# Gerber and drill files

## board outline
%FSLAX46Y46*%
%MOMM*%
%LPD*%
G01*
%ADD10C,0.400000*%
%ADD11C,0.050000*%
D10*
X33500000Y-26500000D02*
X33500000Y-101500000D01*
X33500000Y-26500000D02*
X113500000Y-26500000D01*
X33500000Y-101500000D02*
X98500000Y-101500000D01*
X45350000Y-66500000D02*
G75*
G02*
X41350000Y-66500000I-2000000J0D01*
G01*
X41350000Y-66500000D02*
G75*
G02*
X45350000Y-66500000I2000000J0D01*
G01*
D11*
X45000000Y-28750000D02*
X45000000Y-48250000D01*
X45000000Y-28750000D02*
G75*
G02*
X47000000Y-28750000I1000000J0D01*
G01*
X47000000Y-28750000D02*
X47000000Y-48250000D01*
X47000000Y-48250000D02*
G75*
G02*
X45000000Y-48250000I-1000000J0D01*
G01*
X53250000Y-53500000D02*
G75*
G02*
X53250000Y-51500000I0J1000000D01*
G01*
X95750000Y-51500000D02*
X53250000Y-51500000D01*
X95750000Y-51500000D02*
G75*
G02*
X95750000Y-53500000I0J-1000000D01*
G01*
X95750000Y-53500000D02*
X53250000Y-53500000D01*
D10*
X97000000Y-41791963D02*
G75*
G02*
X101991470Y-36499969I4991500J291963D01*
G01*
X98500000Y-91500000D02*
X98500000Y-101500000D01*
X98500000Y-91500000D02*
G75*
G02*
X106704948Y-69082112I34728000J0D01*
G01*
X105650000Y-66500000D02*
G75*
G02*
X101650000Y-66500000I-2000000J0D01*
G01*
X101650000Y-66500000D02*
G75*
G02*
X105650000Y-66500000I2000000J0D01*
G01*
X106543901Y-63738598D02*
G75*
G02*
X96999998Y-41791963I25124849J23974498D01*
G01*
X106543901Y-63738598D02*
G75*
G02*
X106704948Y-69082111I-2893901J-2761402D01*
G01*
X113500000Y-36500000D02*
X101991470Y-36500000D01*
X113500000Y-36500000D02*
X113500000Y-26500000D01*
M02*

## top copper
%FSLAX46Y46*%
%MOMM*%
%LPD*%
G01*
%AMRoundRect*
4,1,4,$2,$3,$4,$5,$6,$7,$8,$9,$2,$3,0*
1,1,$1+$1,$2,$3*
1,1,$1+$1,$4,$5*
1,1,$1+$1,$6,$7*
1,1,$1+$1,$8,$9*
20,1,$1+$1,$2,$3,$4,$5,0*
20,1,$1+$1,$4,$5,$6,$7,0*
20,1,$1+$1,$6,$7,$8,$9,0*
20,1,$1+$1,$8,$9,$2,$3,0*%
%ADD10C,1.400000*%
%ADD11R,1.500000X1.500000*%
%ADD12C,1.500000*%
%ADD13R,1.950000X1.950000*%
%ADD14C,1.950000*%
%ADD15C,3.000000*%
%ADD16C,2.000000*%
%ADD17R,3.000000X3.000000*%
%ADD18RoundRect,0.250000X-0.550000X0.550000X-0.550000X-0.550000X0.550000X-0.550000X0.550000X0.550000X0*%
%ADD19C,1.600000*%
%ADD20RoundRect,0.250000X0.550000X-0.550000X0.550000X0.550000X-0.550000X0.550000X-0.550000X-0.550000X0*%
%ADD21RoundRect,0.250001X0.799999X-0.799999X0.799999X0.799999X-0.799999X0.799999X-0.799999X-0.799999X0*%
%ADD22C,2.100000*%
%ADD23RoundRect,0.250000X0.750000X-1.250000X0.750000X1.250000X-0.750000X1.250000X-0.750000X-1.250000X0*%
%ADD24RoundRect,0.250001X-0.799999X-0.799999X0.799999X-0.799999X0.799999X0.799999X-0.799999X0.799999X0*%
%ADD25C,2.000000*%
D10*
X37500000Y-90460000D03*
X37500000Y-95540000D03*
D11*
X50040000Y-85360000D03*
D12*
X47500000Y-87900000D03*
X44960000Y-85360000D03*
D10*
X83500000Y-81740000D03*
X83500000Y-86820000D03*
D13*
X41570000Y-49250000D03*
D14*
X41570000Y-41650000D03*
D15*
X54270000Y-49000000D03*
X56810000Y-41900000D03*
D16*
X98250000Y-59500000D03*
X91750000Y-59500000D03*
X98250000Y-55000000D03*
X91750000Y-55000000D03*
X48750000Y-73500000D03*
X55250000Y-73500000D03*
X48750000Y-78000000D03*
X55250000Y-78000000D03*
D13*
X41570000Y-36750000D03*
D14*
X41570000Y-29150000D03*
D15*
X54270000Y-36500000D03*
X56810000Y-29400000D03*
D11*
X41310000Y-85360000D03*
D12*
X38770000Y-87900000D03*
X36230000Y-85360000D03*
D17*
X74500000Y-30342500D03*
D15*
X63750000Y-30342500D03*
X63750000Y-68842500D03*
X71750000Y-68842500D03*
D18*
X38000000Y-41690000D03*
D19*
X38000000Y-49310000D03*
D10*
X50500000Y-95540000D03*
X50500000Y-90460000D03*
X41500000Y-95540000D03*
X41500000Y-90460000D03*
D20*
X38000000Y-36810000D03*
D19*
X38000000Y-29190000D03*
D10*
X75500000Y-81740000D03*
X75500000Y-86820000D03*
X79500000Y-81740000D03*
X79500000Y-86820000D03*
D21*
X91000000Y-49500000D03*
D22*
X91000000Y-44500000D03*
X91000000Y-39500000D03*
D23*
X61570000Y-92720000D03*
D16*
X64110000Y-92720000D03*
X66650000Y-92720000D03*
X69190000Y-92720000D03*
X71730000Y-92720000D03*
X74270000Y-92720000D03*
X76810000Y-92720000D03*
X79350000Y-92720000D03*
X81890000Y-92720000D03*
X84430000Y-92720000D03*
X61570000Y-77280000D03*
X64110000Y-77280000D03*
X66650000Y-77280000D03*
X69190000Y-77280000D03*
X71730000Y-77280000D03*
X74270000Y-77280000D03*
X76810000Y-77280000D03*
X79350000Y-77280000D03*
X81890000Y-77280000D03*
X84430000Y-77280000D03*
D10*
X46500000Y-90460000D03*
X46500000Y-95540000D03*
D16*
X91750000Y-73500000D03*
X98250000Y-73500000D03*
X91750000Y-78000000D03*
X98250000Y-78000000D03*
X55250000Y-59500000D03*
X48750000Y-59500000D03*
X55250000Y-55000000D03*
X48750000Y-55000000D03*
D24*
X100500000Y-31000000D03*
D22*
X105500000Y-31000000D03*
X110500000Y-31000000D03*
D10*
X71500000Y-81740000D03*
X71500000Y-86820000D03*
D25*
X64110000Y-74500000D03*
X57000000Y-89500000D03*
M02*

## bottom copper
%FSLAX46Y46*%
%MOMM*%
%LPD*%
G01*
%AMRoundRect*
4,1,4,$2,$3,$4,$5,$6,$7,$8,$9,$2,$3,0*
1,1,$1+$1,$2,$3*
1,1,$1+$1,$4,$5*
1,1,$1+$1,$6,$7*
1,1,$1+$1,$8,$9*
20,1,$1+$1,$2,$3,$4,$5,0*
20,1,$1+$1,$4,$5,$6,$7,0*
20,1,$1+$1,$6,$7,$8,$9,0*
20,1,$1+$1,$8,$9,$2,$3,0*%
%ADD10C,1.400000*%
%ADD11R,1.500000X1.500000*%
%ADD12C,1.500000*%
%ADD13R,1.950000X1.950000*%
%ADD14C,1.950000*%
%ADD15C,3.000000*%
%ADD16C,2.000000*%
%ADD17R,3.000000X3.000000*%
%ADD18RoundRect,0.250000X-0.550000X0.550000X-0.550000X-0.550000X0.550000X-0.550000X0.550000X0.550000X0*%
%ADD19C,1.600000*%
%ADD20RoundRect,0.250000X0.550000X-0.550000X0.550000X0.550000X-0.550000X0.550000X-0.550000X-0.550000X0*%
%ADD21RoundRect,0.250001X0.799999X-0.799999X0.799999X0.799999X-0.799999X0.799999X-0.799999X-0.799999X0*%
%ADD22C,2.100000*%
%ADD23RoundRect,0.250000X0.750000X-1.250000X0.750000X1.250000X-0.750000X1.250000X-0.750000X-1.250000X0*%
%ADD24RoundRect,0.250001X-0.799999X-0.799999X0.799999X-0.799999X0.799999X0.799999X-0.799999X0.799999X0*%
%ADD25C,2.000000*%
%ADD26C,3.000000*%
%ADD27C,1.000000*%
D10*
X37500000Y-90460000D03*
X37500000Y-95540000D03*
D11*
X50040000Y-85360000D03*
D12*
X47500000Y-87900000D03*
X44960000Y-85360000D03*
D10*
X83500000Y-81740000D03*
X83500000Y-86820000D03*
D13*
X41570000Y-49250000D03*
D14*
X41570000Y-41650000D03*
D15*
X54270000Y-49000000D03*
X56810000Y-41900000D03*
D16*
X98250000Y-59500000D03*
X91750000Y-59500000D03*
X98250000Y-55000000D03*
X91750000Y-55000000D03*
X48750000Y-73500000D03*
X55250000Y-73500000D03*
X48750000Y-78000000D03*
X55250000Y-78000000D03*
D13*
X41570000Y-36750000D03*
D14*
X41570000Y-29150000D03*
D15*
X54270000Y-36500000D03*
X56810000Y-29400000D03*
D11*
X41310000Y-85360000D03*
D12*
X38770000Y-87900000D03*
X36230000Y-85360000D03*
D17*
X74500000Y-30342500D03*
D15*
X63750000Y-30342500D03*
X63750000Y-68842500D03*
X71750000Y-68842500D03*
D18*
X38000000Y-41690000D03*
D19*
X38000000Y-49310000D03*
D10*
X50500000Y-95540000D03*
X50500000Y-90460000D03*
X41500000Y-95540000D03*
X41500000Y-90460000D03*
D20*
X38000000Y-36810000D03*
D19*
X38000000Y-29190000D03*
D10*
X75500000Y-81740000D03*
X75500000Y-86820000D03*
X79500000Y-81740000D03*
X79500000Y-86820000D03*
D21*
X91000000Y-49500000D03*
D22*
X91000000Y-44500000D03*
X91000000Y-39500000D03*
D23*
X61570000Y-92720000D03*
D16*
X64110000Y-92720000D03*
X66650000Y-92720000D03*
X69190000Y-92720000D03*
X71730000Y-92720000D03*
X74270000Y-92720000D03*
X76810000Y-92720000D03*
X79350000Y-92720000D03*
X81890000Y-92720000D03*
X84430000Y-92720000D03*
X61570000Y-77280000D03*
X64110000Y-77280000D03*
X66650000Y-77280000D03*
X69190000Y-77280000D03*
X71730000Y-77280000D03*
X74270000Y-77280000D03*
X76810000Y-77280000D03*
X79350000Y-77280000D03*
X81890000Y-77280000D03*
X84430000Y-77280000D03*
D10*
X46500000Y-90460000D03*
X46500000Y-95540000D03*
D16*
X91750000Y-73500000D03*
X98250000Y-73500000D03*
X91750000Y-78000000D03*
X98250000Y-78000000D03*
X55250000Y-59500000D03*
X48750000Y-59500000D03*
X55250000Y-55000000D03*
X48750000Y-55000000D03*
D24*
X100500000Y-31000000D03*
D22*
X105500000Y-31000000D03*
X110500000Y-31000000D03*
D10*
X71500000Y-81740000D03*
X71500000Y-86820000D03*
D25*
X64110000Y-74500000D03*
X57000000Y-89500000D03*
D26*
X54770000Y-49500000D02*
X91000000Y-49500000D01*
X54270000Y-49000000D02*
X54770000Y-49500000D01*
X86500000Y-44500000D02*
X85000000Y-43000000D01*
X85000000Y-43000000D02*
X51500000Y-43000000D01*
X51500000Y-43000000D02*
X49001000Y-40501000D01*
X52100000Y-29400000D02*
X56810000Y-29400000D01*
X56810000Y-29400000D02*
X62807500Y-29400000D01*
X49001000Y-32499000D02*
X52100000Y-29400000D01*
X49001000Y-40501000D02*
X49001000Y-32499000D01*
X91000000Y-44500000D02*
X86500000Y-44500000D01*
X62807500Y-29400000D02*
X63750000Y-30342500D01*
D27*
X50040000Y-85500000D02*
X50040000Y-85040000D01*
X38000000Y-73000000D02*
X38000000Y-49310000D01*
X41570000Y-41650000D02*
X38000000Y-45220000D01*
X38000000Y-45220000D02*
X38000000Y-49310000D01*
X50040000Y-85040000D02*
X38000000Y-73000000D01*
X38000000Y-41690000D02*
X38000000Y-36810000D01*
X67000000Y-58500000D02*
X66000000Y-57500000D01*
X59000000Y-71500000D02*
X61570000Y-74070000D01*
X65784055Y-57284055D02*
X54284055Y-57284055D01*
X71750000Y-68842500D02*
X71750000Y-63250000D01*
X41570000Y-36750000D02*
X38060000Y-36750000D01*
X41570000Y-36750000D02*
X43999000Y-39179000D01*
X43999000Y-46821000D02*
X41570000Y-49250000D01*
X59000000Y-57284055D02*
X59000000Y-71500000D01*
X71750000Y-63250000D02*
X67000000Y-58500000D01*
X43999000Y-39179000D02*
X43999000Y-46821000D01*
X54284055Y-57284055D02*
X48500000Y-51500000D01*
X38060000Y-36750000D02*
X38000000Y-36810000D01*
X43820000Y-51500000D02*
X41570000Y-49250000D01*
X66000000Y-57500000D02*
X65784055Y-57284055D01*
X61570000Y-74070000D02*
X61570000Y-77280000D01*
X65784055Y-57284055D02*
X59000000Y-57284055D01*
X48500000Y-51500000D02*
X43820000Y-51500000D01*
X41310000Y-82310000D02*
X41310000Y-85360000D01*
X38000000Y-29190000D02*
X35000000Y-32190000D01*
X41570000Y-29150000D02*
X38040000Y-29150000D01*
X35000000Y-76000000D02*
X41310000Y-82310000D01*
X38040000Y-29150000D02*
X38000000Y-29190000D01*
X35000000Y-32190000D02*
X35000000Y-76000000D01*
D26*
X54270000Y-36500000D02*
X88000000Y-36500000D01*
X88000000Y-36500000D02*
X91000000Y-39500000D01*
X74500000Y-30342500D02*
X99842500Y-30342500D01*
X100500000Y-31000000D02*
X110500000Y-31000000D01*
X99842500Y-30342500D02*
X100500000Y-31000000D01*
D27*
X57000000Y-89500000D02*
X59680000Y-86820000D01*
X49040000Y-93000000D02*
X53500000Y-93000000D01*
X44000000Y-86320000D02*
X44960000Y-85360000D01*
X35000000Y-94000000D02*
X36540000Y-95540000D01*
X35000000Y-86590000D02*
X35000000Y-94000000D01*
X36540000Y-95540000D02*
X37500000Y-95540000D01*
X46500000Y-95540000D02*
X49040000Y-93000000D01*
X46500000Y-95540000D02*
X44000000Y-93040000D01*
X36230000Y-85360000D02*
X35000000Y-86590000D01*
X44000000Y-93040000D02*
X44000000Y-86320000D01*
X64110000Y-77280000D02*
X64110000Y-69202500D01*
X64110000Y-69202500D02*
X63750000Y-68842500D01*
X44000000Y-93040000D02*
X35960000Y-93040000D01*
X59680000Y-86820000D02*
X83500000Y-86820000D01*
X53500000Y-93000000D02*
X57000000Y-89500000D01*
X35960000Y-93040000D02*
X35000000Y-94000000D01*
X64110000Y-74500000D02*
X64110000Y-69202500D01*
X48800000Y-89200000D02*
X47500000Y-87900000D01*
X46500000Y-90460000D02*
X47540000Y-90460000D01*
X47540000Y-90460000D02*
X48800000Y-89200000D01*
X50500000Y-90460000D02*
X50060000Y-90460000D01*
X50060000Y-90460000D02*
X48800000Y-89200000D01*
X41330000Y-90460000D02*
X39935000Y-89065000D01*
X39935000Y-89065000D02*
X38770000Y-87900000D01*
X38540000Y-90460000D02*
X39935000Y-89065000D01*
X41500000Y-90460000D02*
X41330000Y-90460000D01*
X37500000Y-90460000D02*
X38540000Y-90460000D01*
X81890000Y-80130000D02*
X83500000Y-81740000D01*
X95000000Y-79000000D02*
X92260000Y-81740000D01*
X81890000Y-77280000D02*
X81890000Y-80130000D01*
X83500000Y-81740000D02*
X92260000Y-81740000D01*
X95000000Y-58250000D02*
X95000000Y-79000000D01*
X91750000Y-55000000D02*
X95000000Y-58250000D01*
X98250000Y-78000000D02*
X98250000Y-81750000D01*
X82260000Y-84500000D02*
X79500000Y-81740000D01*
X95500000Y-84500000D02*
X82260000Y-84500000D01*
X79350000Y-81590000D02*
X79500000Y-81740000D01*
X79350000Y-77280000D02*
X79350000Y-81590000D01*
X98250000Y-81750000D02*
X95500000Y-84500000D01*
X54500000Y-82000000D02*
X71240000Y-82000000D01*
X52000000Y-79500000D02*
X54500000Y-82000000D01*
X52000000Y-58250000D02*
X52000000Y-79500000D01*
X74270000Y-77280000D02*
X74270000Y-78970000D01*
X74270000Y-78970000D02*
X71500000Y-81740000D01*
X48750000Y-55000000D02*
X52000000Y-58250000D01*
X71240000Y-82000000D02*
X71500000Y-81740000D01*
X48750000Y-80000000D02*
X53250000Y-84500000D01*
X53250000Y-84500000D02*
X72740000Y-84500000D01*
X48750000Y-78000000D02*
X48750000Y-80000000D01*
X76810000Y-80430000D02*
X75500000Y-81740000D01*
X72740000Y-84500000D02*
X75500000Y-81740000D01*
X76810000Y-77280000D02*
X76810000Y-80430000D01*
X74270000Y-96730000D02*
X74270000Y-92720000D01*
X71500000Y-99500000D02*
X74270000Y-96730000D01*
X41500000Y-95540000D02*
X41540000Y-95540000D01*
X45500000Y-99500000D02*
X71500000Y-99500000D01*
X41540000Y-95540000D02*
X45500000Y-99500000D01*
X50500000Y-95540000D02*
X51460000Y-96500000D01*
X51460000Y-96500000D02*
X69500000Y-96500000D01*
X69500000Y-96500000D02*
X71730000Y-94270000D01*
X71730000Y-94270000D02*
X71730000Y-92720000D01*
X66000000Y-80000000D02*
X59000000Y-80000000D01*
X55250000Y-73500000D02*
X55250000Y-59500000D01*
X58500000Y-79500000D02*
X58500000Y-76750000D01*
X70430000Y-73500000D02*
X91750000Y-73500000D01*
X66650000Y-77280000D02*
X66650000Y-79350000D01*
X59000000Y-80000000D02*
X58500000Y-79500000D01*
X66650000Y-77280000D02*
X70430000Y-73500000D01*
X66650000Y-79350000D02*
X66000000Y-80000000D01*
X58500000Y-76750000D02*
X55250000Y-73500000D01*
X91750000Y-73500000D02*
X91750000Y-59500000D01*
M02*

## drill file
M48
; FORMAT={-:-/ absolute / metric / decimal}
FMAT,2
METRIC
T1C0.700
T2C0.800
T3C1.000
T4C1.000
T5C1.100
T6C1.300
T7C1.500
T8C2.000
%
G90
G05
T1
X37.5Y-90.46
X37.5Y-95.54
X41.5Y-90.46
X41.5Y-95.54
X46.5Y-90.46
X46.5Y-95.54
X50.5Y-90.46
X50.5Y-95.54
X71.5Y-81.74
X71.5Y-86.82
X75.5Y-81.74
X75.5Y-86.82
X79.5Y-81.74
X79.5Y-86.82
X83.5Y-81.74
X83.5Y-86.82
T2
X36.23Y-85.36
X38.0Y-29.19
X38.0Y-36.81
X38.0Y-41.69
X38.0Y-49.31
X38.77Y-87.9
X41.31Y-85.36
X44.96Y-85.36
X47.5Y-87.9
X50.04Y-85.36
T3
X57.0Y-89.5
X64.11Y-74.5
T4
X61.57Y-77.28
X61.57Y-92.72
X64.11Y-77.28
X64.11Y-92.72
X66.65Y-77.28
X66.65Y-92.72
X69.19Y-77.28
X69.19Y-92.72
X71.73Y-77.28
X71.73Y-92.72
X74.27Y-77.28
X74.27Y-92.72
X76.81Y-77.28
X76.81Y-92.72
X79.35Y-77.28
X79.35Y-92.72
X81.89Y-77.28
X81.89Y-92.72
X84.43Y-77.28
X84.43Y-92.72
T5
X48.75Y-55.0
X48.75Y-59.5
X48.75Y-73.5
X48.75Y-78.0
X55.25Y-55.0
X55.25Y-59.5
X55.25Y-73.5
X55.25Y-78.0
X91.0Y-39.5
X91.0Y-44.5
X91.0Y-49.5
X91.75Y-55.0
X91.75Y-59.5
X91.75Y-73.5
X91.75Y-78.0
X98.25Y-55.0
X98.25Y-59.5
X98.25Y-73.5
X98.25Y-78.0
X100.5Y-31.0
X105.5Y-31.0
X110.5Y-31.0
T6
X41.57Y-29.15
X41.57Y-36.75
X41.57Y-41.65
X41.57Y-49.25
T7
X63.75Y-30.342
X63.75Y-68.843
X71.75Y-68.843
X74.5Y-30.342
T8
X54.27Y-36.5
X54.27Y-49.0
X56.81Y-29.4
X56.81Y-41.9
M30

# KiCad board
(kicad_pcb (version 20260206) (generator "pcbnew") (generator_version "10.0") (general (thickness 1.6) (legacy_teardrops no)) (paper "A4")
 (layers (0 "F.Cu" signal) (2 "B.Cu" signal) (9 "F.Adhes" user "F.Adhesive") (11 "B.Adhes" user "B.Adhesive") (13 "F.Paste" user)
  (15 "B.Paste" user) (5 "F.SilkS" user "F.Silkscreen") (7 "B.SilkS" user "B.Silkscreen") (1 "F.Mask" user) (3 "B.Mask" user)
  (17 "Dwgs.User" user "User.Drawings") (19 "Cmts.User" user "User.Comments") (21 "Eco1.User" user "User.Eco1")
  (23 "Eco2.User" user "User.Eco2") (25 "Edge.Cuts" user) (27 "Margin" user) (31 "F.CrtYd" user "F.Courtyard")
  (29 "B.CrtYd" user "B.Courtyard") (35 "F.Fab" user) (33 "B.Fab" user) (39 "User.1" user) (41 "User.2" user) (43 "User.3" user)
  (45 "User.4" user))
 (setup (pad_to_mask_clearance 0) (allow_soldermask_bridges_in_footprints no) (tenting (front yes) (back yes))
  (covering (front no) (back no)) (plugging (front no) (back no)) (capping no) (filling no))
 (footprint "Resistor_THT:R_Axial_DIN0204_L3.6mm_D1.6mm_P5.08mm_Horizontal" (layer "F.Cu") (at 37.5 90.46 -90)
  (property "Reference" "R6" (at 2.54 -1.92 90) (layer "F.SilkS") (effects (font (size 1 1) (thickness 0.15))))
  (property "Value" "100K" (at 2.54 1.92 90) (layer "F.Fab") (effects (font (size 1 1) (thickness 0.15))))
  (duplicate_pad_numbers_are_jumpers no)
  (pad "1" thru_hole circle (at 0 0 270) (size 1.4 1.4) (drill 0.7) (layers "*.Cu" "*.Mask") (remove_unused_layers no) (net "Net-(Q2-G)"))
  (pad "2" thru_hole circle (at 5.08 0 270) (size 1.4 1.4) (drill 0.7) (layers "*.Cu" "*.Mask") (remove_unused_layers no) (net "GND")))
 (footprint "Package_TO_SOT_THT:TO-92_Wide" (layer "F.Cu") (at 50.04 85.36 180)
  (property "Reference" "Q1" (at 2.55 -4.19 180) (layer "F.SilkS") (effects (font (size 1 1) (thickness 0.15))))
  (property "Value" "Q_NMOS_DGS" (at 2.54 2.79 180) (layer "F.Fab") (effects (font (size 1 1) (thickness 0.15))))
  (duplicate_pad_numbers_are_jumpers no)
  (pad "1" thru_hole rect (at 0 0 180) (size 1.5 1.5) (drill 0.8) (layers "*.Cu" "*.Mask") (remove_unused_layers no) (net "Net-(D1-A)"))
  (pad "2" thru_hole circle (at 2.54 -2.54 180) (size 1.5 1.5) (drill 0.8) (layers "*.Cu" "*.Mask") (remove_unused_layers no)
   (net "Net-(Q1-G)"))
  (pad "3" thru_hole circle (at 5.08 0 180) (size 1.5 1.5) (drill 0.8) (layers "*.Cu" "*.Mask") (remove_unused_layers no) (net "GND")))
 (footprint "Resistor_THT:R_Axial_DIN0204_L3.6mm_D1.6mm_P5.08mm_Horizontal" (layer "F.Cu") (at 83.5 81.74 -90)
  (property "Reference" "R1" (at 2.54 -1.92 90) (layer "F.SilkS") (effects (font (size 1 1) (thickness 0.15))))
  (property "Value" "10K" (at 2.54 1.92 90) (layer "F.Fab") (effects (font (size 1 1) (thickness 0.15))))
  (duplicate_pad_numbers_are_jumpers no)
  (pad "1" thru_hole circle (at 0 0 270) (size 1.4 1.4) (drill 0.7) (layers "*.Cu" "*.Mask") (remove_unused_layers no) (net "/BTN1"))
  (pad "2" thru_hole circle (at 5.08 0 270) (size 1.4 1.4) (drill 0.7) (layers "*.Cu" "*.Mask") (remove_unused_layers no) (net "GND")))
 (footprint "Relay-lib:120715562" (layer "F.Cu") (at 41.57 49.25)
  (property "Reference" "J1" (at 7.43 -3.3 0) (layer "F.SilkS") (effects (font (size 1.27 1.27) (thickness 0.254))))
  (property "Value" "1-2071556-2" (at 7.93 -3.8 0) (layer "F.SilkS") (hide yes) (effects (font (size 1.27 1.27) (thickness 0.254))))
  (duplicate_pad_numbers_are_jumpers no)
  (pad "1" thru_hole rect (at 0 0) (size 1.95 1.95) (drill 1.3) (layers "*.Cu" "*.Mask") (remove_unused_layers no) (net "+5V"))
  (pad "2" thru_hole circle (at 0 -7.6) (size 1.95 1.95) (drill 1.3) (layers "*.Cu" "*.Mask") (remove_unused_layers no) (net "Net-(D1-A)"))
  (pad "3" thru_hole circle (at 12.7 -0.25) (size 3 3) (drill 2) (layers "*.Cu" "*.Mask") (remove_unused_layers no) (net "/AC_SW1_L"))
  (pad "4" thru_hole circle (at 15.24 -7.35) (size 3 3) (drill 2) (layers "*.Cu" "*.Mask") (remove_unused_layers no) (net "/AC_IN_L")))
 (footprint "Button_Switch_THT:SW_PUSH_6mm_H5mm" (layer "F.Cu") (at 98.25 59.5 180)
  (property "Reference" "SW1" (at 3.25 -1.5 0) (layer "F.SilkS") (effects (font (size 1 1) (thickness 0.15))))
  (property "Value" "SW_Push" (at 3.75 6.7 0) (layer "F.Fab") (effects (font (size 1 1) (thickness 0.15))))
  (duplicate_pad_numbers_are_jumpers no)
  (pad "1" thru_hole circle (at 0 0 270) (size 2 2) (drill 1.1) (layers "*.Cu" "*.Mask") (remove_unused_layers no) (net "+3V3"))
  (pad "1" thru_hole circle (at 6.5 0 270) (size 2 2) (drill 1.1) (layers "*.Cu" "*.Mask") (remove_unused_layers no) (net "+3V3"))
  (pad "2" thru_hole circle (at 0 4.5 270) (size 2 2) (drill 1.1) (layers "*.Cu" "*.Mask") (remove_unused_layers no) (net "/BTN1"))
  (pad "2" thru_hole circle (at 6.5 4.5 270) (size 2 2) (drill 1.1) (layers "*.Cu" "*.Mask") (remove_unused_layers no) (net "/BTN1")))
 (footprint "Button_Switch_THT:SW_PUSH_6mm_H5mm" (layer "F.Cu") (at 48.75 73.5)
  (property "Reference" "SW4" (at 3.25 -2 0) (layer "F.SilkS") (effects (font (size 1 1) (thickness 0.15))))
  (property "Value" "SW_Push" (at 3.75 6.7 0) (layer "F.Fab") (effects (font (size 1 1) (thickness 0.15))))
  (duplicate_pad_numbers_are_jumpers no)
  (pad "1" thru_hole circle (at 0 0 90) (size 2 2) (drill 1.1) (layers "*.Cu" "*.Mask") (remove_unused_layers no) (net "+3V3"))
  (pad "1" thru_hole circle (at 6.5 0 90) (size 2 2) (drill 1.1) (layers "*.Cu" "*.Mask") (remove_unused_layers no) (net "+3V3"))
  (pad "2" thru_hole circle (at 0 4.5 90) (size 2 2) (drill 1.1) (layers "*.Cu" "*.Mask") (remove_unused_layers no) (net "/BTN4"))
  (pad "2" thru_hole circle (at 6.5 4.5 90) (size 2 2) (drill 1.1) (layers "*.Cu" "*.Mask") (remove_unused_layers no) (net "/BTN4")))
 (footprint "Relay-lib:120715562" (layer "F.Cu") (at 41.57 36.75)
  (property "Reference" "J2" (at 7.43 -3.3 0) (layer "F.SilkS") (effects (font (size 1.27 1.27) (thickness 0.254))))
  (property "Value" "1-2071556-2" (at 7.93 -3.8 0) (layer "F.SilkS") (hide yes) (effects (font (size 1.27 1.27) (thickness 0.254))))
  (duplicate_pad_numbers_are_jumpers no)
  (pad "1" thru_hole rect (at 0 0) (size 1.95 1.95) (drill 1.3) (layers "*.Cu" "*.Mask") (remove_unused_layers no) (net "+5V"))
  (pad "2" thru_hole circle (at 0 -7.6) (size 1.95 1.95) (drill 1.3) (layers "*.Cu" "*.Mask") (remove_unused_layers no) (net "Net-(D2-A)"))
  (pad "3" thru_hole circle (at 12.7 -0.25) (size 3 3) (drill 2) (layers "*.Cu" "*.Mask") (remove_unused_layers no) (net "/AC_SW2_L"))
  (pad "4" thru_hole circle (at 15.24 -7.35) (size 3 3) (drill 2) (layers "*.Cu" "*.Mask") (remove_unused_layers no) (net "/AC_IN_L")))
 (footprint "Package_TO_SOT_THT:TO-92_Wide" (layer "F.Cu") (at 41.31 85.36 180)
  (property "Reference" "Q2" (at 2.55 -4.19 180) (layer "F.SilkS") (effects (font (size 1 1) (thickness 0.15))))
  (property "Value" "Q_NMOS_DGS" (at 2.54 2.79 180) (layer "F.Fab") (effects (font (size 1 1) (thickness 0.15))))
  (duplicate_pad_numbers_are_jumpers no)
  (pad "1" thru_hole rect (at 0 0 180) (size 1.5 1.5) (drill 0.8) (layers "*.Cu" "*.Mask") (remove_unused_layers no) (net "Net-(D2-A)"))
  (pad "2" thru_hole circle (at 2.54 -2.54 180) (size 1.5 1.5) (drill 0.8) (layers "*.Cu" "*.Mask") (remove_unused_layers no)
   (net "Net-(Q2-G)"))
  (pad "3" thru_hole circle (at 5.08 0 180) (size 1.5 1.5) (drill 0.8) (layers "*.Cu" "*.Mask") (remove_unused_layers no) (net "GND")))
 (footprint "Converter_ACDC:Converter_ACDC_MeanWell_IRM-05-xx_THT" (layer "F.Cu") (at 74.5 30.3425 -90)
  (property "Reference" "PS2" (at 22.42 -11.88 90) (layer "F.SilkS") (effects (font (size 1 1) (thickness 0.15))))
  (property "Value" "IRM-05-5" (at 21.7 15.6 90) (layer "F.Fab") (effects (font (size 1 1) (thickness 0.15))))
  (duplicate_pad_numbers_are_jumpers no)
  (pad "1" thru_hole rect (at 0 0 270) (size 3 3) (drill 1.5) (layers "*.Cu" "*.Mask") (remove_unused_layers no) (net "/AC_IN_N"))
  (pad "2" thru_hole circle (at 0 10.75 270) (size 3 3) (drill 1.5) (layers "*.Cu" "*.Mask") (remove_unused_layers no) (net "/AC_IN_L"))
  (pad "3" thru_hole circle (at 38.5 10.75 270) (size 3 3) (drill 1.5) (layers "*.Cu" "*.Mask") (remove_unused_layers no) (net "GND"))
  (pad "4" thru_hole circle (at 38.5 2.75 270) (size 3 3) (drill 1.5) (layers "*.Cu" "*.Mask") (remove_unused_layers no) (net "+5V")))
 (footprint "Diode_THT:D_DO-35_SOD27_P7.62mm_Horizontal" (layer "F.Cu") (at 38 41.69 -90)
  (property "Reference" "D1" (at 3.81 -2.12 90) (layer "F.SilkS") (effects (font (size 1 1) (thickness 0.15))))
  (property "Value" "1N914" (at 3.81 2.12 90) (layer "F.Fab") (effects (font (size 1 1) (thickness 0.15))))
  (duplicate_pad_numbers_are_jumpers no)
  (pad "1" thru_hole roundrect (at 0 0 270) (size 1.6 1.6) (drill 0.8) (layers "*.Cu" "*.Mask") (remove_unused_layers no)
   (roundrect_rratio 0.15625) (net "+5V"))
  (pad "2" thru_hole circle (at 7.62 0 270) (size 1.6 1.6) (drill 0.8) (layers "*.Cu" "*.Mask") (remove_unused_layers no) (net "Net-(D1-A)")))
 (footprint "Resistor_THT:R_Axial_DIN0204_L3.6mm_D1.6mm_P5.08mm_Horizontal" (layer "F.Cu") (at 50.5 95.54 90)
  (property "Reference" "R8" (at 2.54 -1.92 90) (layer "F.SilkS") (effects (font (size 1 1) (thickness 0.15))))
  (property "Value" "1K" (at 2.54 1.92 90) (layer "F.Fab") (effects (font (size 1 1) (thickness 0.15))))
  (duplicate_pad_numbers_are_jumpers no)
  (pad "1" thru_hole circle (at 0 0 90) (size 1.4 1.4) (drill 0.7) (layers "*.Cu" "*.Mask") (remove_unused_layers no) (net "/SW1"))
  (pad "2" thru_hole circle (at 5.08 0 90) (size 1.4 1.4) (drill 0.7) (layers "*.Cu" "*.Mask") (remove_unused_layers no) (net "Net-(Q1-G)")))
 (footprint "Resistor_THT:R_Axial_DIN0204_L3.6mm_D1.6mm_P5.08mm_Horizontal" (layer "F.Cu") (at 41.5 95.54 90)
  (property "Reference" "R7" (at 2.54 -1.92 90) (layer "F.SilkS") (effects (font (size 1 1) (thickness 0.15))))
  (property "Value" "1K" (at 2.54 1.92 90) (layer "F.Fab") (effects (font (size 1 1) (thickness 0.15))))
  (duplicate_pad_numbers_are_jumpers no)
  (pad "1" thru_hole circle (at 0 0 90) (size 1.4 1.4) (drill 0.7) (layers "*.Cu" "*.Mask") (remove_unused_layers no) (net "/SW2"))
  (pad "2" thru_hole circle (at 5.08 0 90) (size 1.4 1.4) (drill 0.7) (layers "*.Cu" "*.Mask") (remove_unused_layers no) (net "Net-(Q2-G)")))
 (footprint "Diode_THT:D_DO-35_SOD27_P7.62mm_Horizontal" (layer "F.Cu") (at 38 36.81 90)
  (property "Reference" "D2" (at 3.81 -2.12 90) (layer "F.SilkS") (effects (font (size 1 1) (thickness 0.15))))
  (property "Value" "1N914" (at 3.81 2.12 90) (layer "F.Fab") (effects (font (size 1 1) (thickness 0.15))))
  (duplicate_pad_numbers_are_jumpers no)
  (pad "1" thru_hole roundrect (at 0 0 90) (size 1.6 1.6) (drill 0.8) (layers "*.Cu" "*.Mask") (remove_unused_layers no)
   (roundrect_rratio 0.15625) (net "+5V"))
  (pad "2" thru_hole circle (at 7.62 0 90) (size 1.6 1.6) (drill 0.8) (layers "*.Cu" "*.Mask") (remove_unused_layers no) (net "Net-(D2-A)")))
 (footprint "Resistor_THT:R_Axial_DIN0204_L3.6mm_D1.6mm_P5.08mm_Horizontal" (layer "F.Cu") (at 75.5 81.74 -90)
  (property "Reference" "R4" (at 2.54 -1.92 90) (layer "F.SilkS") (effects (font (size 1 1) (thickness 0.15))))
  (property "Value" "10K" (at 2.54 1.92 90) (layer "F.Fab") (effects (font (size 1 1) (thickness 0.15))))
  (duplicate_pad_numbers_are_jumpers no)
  (pad "1" thru_hole circle (at 0 0 270) (size 1.4 1.4) (drill 0.7) (layers "*.Cu" "*.Mask") (remove_unused_layers no) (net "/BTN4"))
  (pad "2" thru_hole circle (at 5.08 0 270) (size 1.4 1.4) (drill 0.7) (layers "*.Cu" "*.Mask") (remove_unused_layers no) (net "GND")))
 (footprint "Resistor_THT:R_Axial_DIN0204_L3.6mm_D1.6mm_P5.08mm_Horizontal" (layer "F.Cu") (at 79.5 81.74 -90)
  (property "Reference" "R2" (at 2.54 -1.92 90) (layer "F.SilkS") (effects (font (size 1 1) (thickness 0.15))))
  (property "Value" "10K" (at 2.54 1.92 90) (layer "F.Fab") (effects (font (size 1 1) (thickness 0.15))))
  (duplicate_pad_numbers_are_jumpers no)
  (pad "1" thru_hole circle (at 0 0 270) (size 1.4 1.4) (drill 0.7) (layers "*.Cu" "*.Mask") (remove_unused_layers no) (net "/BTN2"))
  (pad "2" thru_hole circle (at 5.08 0 270) (size 1.4 1.4) (drill 0.7) (layers "*.Cu" "*.Mask") (remove_unused_layers no) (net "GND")))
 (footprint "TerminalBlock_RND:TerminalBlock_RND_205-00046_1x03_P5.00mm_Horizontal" (layer "F.Cu") (at 91 49.5 90)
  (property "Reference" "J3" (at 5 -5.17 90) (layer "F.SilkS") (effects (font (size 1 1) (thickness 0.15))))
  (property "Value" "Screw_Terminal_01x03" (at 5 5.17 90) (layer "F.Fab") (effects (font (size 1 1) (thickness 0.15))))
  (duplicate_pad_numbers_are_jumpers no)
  (pad "1" thru_hole roundrect (at 0 0 90) (size 2.1 2.1) (drill 1.1) (layers "*.Cu" "*.Mask") (remove_unused_layers no)
   (roundrect_rratio 0.119048) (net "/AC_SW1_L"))
  (pad "2" thru_hole circle (at 5 0 90) (size 2.1 2.1) (drill 1.1) (layers "*.Cu" "*.Mask") (remove_unused_layers no) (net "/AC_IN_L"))
  (pad "3" thru_hole circle (at 10 0 90) (size 2.1 2.1) (drill 1.1) (layers "*.Cu" "*.Mask") (remove_unused_layers no) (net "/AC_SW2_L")))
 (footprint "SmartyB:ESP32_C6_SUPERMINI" (layer "F.Cu") (at 73 85 90)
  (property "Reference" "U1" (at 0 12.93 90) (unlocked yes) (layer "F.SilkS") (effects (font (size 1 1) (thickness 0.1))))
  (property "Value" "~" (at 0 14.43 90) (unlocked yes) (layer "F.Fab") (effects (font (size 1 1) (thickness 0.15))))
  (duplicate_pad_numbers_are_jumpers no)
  (pad "1" thru_hole roundrect (at -7.72 -11.43 90) (size 3 2) (drill 1) (layers "*.Cu" "*.Mask") (remove_unused_layers no)
   (roundrect_rratio 0.125) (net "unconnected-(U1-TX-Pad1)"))
  (pad "2" thru_hole circle (at -7.72 -8.89 90) (size 2 2) (drill 1) (layers "*.Cu" "*.Mask") (remove_unused_layers no)
   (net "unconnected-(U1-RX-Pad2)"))
  (pad "3" thru_hole circle (at -7.72 -6.35 90) (size 2 2) (drill 1) (layers "*.Cu" "*.Mask") (remove_unused_layers no)
   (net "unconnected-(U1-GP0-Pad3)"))
  (pad "4" thru_hole circle (at -7.72 -3.81 90) (size 2 2) (drill 1) (layers "*.Cu" "*.Mask") (remove_unused_layers no)
   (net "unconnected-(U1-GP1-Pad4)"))
  (pad "5" thru_hole circle (at -7.72 -1.27 90) (size 2 2) (drill 1) (layers "*.Cu" "*.Mask") (remove_unused_layers no) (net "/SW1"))
  (pad "6" thru_hole circle (at -7.72 1.27 90) (size 2 2) (drill 1) (layers "*.Cu" "*.Mask") (remove_unused_layers no) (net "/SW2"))
  (pad "7" thru_hole circle (at -7.72 3.81 90) (size 2 2) (drill 1) (layers "*.Cu" "*.Mask") (remove_unused_layers no)
   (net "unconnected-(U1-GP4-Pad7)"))
  (pad "8" thru_hole circle (at -7.72 6.35 90) (size 2 2) (drill 1) (layers "*.Cu" "*.Mask") (remove_unused_layers no)
   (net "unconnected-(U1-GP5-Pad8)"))
  (pad "9" thru_hole circle (at -7.72 8.89 90) (size 2 2) (drill 1) (layers "*.Cu" "*.Mask") (remove_unused_layers no)
   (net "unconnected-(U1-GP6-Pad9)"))
  (pad "10" thru_hole circle (at -7.72 11.43 90) (size 2 2) (drill 1) (layers "*.Cu" "*.Mask") (remove_unused_layers no)
   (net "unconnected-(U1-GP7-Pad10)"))
  (pad "11" thru_hole circle (at 7.72 -11.43 90) (size 2 2) (drill 1) (layers "*.Cu" "*.Mask") (remove_unused_layers no) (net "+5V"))
  (pad "12" thru_hole circle (at 7.72 -8.89 90) (size 2 2) (drill 1) (layers "*.Cu" "*.Mask") (remove_unused_layers no) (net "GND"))
  (pad "13" thru_hole circle (at 7.72 -6.35 90) (size 2 2) (drill 1) (layers "*.Cu" "*.Mask") (remove_unused_layers no) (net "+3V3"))
  (pad "14" thru_hole circle (at 7.72 -3.81 90) (size 2 2) (drill 1) (layers "*.Cu" "*.Mask") (remove_unused_layers no)
   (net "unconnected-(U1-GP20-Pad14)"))
  (pad "15" thru_hole circle (at 7.72 -1.27 90) (size 2 2) (drill 1) (layers "*.Cu" "*.Mask") (remove_unused_layers no)
   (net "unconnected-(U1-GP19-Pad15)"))
  (pad "16" thru_hole circle (at 7.72 1.27 90) (size 2 2) (drill 1) (layers "*.Cu" "*.Mask") (remove_unused_layers no) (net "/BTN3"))
  (pad "17" thru_hole circle (at 7.72 3.81 90) (size 2 2) (drill 1) (layers "*.Cu" "*.Mask") (remove_unused_layers no) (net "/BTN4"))
  (pad "18" thru_hole circle (at 7.72 6.35 90) (size 2 2) (drill 1) (layers "*.Cu" "*.Mask") (remove_unused_layers no) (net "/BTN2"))
  (pad "19" thru_hole circle (at 7.72 8.89 90) (size 2 2) (drill 1) (layers "*.Cu" "*.Mask") (remove_unused_layers no) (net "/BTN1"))
  (pad "20" thru_hole circle (at 7.72 11.43 90) (size 2 2) (drill 1) (layers "*.Cu" "*.Mask") (remove_unused_layers no)
   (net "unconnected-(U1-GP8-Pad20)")))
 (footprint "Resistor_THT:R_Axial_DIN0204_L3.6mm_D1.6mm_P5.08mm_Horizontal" (layer "F.Cu") (at 46.5 90.46 -90)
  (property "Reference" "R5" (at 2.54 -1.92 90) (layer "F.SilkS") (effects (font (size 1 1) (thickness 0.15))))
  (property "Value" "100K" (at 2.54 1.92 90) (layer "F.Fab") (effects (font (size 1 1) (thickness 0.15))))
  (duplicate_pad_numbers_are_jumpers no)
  (pad "1" thru_hole circle (at 0 0 270) (size 1.4 1.4) (drill 0.7) (layers "*.Cu" "*.Mask") (remove_unused_layers no) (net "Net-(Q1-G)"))
  (pad "2" thru_hole circle (at 5.08 0 270) (size 1.4 1.4) (drill 0.7) (layers "*.Cu" "*.Mask") (remove_unused_layers no) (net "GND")))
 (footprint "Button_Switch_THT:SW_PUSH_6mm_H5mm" (layer "F.Cu") (at 91.75 73.5)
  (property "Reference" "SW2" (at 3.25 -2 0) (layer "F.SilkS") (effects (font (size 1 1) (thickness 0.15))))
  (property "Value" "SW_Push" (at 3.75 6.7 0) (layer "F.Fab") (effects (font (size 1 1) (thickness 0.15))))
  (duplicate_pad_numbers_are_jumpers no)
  (pad "1" thru_hole circle (at 0 0 90) (size 2 2) (drill 1.1) (layers "*.Cu" "*.Mask") (remove_unused_layers no) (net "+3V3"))
  (pad "1" thru_hole circle (at 6.5 0 90) (size 2 2) (drill 1.1) (layers "*.Cu" "*.Mask") (remove_unused_layers no) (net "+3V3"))
  (pad "2" thru_hole circle (at 0 4.5 90) (size 2 2) (drill 1.1) (layers "*.Cu" "*.Mask") (remove_unused_layers no) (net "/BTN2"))
  (pad "2" thru_hole circle (at 6.5 4.5 90) (size 2 2) (drill 1.1) (layers "*.Cu" "*.Mask") (remove_unused_layers no) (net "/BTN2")))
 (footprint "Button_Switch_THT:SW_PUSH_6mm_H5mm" (layer "F.Cu") (at 55.25 59.5 180)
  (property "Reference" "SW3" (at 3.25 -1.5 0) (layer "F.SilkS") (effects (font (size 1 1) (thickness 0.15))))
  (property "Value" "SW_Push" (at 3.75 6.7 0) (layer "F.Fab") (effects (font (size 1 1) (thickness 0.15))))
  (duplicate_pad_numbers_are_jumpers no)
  (pad "1" thru_hole circle (at 0 0 270) (size 2 2) (drill 1.1) (layers "*.Cu" "*.Mask") (remove_unused_layers no) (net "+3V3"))
  (pad "1" thru_hole circle (at 6.5 0 270) (size 2 2) (drill 1.1) (layers "*.Cu" "*.Mask") (remove_unused_layers no) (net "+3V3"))
  (pad "2" thru_hole circle (at 0 4.5 270) (size 2 2) (drill 1.1) (layers "*.Cu" "*.Mask") (remove_unused_layers no) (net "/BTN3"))
  (pad "2" thru_hole circle (at 6.5 4.5 270) (size 2 2) (drill 1.1) (layers "*.Cu" "*.Mask") (remove_unused_layers no) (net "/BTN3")))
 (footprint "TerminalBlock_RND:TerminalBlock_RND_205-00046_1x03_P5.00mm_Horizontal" (layer "F.Cu") (at 100.5 31)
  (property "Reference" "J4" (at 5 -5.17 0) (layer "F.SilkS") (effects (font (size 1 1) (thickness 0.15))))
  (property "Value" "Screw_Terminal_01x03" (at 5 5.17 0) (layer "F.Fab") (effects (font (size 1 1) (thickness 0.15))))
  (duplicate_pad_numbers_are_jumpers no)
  (pad "1" thru_hole roundrect (at 0 0) (size 2.1 2.1) (drill 1.1) (layers "*.Cu" "*.Mask") (remove_unused_layers no)
   (roundrect_rratio 0.119048) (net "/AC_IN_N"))
  (pad "2" thru_hole circle (at 5 0) (size 2.1 2.1) (drill 1.1) (layers "*.Cu" "*.Mask") (remove_unused_layers no) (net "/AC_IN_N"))
  (pad "3" thru_hole circle (at 10 0) (size 2.1 2.1) (drill 1.1) (layers "*.Cu" "*.Mask") (remove_unused_layers no) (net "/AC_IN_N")))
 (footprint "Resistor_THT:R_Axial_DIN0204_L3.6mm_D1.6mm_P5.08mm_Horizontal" (layer "F.Cu") (at 71.5 81.74 -90)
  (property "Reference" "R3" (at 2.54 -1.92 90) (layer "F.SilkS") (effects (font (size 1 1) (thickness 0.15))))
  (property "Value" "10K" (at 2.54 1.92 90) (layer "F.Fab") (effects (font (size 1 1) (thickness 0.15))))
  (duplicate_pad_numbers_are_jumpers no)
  (pad "1" thru_hole circle (at 0 0 270) (size 1.4 1.4) (drill 0.7) (layers "*.Cu" "*.Mask") (remove_unused_layers no) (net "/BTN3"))
  (pad "2" thru_hole circle (at 5.08 0 270) (size 1.4 1.4) (drill 0.7) (layers "*.Cu" "*.Mask") (remove_unused_layers no) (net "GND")))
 (gr_line (start 33.5 26.5) (end 33.5 101.5) (stroke (width 0.4) (type default)) (layer "Edge.Cuts"))
 (gr_line (start 33.5 26.5) (end 113.5 26.5) (stroke (width 0.4) (type default)) (layer "Edge.Cuts"))
 (gr_line (start 33.5 101.5) (end 98.5 101.5) (stroke (width 0.4) (type default)) (layer "Edge.Cuts"))
 (gr_circle (center 43.35 66.5) (end 45.35 66.5) (stroke (width 0.4) (type default)) (fill no) (layer "Edge.Cuts"))
 (gr_line (start 45 28.75) (end 45 48.25) (stroke (width 0.05) (type default)) (layer "Edge.Cuts"))
 (gr_arc (start 45 28.75) (mid 46 27.75) (end 47 28.75) (stroke (width 0.05) (type default)) (layer "Edge.Cuts"))
 (gr_line (start 47 28.75) (end 47 48.25) (stroke (width 0.05) (type default)) (layer "Edge.Cuts"))
 (gr_arc (start 47 48.25) (mid 46 49.25) (end 45 48.25) (stroke (width 0.05) (type default)) (layer "Edge.Cuts"))
 (gr_arc (start 53.25 53.5) (mid 52.25 52.5) (end 53.25 51.5) (stroke (width 0.05) (type default)) (layer "Edge.Cuts"))
 (gr_line (start 95.75 51.5) (end 53.25 51.5) (stroke (width 0.05) (type default)) (layer "Edge.Cuts"))
 (gr_arc (start 95.75 51.5) (mid 96.75 52.5) (end 95.75 53.5) (stroke (width 0.05) (type default)) (layer "Edge.Cuts"))
 (gr_line (start 95.75 53.5) (end 53.25 53.5) (stroke (width 0.05) (type default)) (layer "Edge.Cuts"))
 (gr_arc (start 97 41.791963) (mid 98.354174 38.069243) (end 101.99147 36.5) (stroke (width 0.4) (type default)) (layer "Edge.Cuts"))
 (gr_line (start 98.5 91.5) (end 98.5 101.5) (stroke (width 0.4) (type default)) (layer "Edge.Cuts"))
 (gr_arc (start 98.5 91.5) (mid 100.615682 79.56389) (end 106.704947 69.082111) (stroke (width 0.4) (type default)) (layer "Edge.Cuts"))
 (gr_circle (center 103.65 66.5) (end 105.65 66.5) (stroke (width 0.4) (type default)) (fill no) (layer "Edge.Cuts"))
 (gr_arc (start 106.543901 63.738598) (mid 99.821736 53.613368) (end 97 41.791963) (stroke (width 0.4) (type default)) (layer "Edge.Cuts"))
 (gr_arc (start 106.543901 63.738598) (mid 107.648185 66.3795) (end 106.704947 69.082111) (stroke (width 0.4) (type default))
  (layer "Edge.Cuts"))
 (gr_line (start 113.5 36.5) (end 101.99147 36.5) (stroke (width 0.4) (type default)) (layer "Edge.Cuts"))
 (gr_line (start 113.5 36.5) (end 113.5 26.5) (stroke (width 0.4) (type default)) (layer "Edge.Cuts"))
 (segment (start 54.77 49.5) (end 91 49.5) (width 3) (layer "B.Cu") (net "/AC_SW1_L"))
 (segment (start 54.27 49) (end 54.77 49.5) (width 3) (layer "B.Cu") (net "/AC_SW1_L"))
 (segment (start 86.5 44.5) (end 85 43) (width 3) (layer "B.Cu") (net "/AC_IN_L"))
 (segment (start 85 43) (end 51.5 43) (width 3) (layer "B.Cu") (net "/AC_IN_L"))
 (segment (start 51.5 43) (end 49.001 40.501) (width 3) (layer "B.Cu") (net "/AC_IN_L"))
 (segment (start 52.1 29.4) (end 56.81 29.4) (width 3) (layer "B.Cu") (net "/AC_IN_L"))
 (segment (start 56.81 29.4) (end 62.8075 29.4) (width 3) (layer "B.Cu") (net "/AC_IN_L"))
 (segment (start 49.001 32.499) (end 52.1 29.4) (width 3) (layer "B.Cu") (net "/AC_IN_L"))
 (segment (start 49.001 40.501) (end 49.001 32.499) (width 3) (layer "B.Cu") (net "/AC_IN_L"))
 (segment (start 91 44.5) (end 86.5 44.5) (width 3) (layer "B.Cu") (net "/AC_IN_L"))
 (segment (start 62.8075 29.4) (end 63.75 30.3425) (width 3) (layer "B.Cu") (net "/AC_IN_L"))
 (segment (start 50.04 85.5) (end 50.04 85.04) (width 1) (layer "B.Cu") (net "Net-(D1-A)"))
 (segment (start 38 73) (end 38 49.31) (width 1) (layer "B.Cu") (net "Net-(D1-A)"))
 (segment (start 41.57 41.65) (end 38 45.22) (width 1) (layer "B.Cu") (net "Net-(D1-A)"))
 (segment (start 38 45.22) (end 38 49.31) (width 1) (layer "B.Cu") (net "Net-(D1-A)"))
 (segment (start 50.04 85.04) (end 38 73) (width 1) (layer "B.Cu") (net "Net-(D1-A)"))
 (segment (start 38 41.69) (end 38 36.81) (width 1) (layer "B.Cu") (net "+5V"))
 (segment (start 67 58.5) (end 66 57.5) (width 1) (layer "B.Cu") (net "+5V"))
 (segment (start 59 71.5) (end 61.57 74.07) (width 1) (layer "B.Cu") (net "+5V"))
 (segment (start 65.784055 57.284055) (end 54.284055 57.284055) (width 1) (layer "B.Cu") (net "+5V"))
 (segment (start 71.75 68.8425) (end 71.75 63.25) (width 1) (layer "B.Cu") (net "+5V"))
 (segment (start 41.57 36.75) (end 38.06 36.75) (width 1) (layer "B.Cu") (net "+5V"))
 (segment (start 41.57 36.75) (end 43.999 39.179) (width 1) (layer "B.Cu") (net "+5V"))
 (segment (start 43.999 46.821) (end 41.57 49.25) (width 1) (layer "B.Cu") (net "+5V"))
 (segment (start 59 57.284055) (end 59 71.5) (width 1) (layer "B.Cu") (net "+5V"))
 (segment (start 71.75 63.25) (end 67 58.5) (width 1) (layer "B.Cu") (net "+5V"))
 (segment (start 43.999 39.179) (end 43.999 46.821) (width 1) (layer "B.Cu") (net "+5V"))
 (segment (start 54.284055 57.284055) (end 48.5 51.5) (width 1) (layer "B.Cu") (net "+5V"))
 (segment (start 38.06 36.75) (end 38 36.81) (width 1) (layer "B.Cu") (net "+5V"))
 (segment (start 43.82 51.5) (end 41.57 49.25) (width 1) (layer "B.Cu") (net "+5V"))
 (segment (start 66 57.5) (end 65.784055 57.284055) (width 1) (layer "B.Cu") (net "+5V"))
 (segment (start 61.57 74.07) (end 61.57 77.28) (width 1) (layer "B.Cu") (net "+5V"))
 (segment (start 65.784055 57.284055) (end 59 57.284055) (width 1) (layer "B.Cu") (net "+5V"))
 (segment (start 48.5 51.5) (end 43.82 51.5) (width 1) (layer "B.Cu") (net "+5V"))
 (segment (start 41.31 82.31) (end 41.31 85.36) (width 1) (layer "B.Cu") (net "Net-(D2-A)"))
 (segment (start 38 29.19) (end 35 32.19) (width 1) (layer "B.Cu") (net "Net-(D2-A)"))
 (segment (start 41.57 29.15) (end 38.04 29.15) (width 1) (layer "B.Cu") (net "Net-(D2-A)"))
 (segment (start 35 76) (end 41.31 82.31) (width 1) (layer "B.Cu") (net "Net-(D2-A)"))
 (segment (start 38.04 29.15) (end 38 29.19) (width 1) (layer "B.Cu") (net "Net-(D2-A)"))
 (segment (start 35 32.19) (end 35 76) (width 1) (layer "B.Cu") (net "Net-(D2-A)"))
 (segment (start 54.27 36.5) (end 88 36.5) (width 3) (layer "B.Cu") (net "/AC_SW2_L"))
 (segment (start 88 36.5) (end 91 39.5) (width 3) (layer "B.Cu") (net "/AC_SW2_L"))
 (segment (start 74.5 30.3425) (end 99.8425 30.3425) (width 3) (layer "B.Cu") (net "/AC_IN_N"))
 (segment (start 100.5 31) (end 110.5 31) (width 3) (layer "B.Cu") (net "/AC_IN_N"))
 (segment (start 99.8425 30.3425) (end 100.5 31) (width 3) (layer "B.Cu") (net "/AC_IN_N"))
 (via (at 64.11 74.5) (size 2) (drill 1) (layers "F.Cu" "B.Cu") (capping no) (covering (front no) (back no)) (plugging (front no) (back no))
  (filling no) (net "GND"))
 (via (at 57 89.5) (size 2) (drill 1) (layers "F.Cu" "B.Cu") (capping no) (covering (front no) (back no)) (plugging (front no) (back no))
  (filling no) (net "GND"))
 (segment (start 57 89.5) (end 59.68 86.82) (width 1) (layer "B.Cu") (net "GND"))
 (segment (start 49.04 93) (end 53.5 93) (width 1) (layer "B.Cu") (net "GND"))
 (segment (start 44 86.32) (end 44.96 85.36) (width 1) (layer "B.Cu") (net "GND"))
 (segment (start 35 94) (end 36.54 95.54) (width 1) (layer "B.Cu") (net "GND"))
 (segment (start 35 86.59) (end 35 94) (width 1) (layer "B.Cu") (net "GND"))
 (segment (start 36.54 95.54) (end 37.5 95.54) (width 1) (layer "B.Cu") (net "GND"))
 (segment (start 46.5 95.54) (end 49.04 93) (width 1) (layer "B.Cu") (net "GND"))
 (segment (start 46.5 95.54) (end 44 93.04) (width 1) (layer "B.Cu") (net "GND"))
 (segment (start 36.23 85.36) (end 35 86.59) (width 1) (layer "B.Cu") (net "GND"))
 (segment (start 44 93.04) (end 44 86.32) (width 1) (layer "B.Cu") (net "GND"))
 (segment (start 64.11 77.28) (end 64.11 69.2025) (width 1) (layer "B.Cu") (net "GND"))
 (segment (start 64.11 69.2025) (end 63.75 68.8425) (width 1) (layer "B.Cu") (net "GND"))
 (segment (start 44 93.04) (end 35.96 93.04) (width 1) (layer "B.Cu") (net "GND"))
 (segment (start 59.68 86.82) (end 83.5 86.82) (width 1) (layer "B.Cu") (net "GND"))
 (segment (start 53.5 93) (end 57 89.5) (width 1) (layer "B.Cu") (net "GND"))
 (segment (start 35.96 93.04) (end 35 94) (width 1) (layer "B.Cu") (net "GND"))
 (segment (start 64.11 74.5) (end 64.11 69.2025) (width 1) (layer "B.Cu") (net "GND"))
 (segment (start 48.8 89.2) (end 47.5 87.9) (width 1) (layer "B.Cu") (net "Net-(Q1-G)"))
 (segment (start 46.5 90.46) (end 47.54 90.46) (width 1) (layer "B.Cu") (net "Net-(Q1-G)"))
 (segment (start 47.54 90.46) (end 48.8 89.2) (width 1) (layer "B.Cu") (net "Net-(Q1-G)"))
 (segment (start 50.5 90.46) (end 50.06 90.46) (width 1) (layer "B.Cu") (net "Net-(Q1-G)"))
 (segment (start 50.06 90.46) (end 48.8 89.2) (width 1) (layer "B.Cu") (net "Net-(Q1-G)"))
 (segment (start 41.33 90.46) (end 39.935 89.065) (width 1) (layer "B.Cu") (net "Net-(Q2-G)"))
 (segment (start 39.935 89.065) (end 38.77 87.9) (width 1) (layer "B.Cu") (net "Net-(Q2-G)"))
 (segment (start 38.54 90.46) (end 39.935 89.065) (width 1) (layer "B.Cu") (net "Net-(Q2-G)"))
 (segment (start 41.5 90.46) (end 41.33 90.46) (width 1) (layer "B.Cu") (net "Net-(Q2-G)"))
 (segment (start 37.5 90.46) (end 38.54 90.46) (width 1) (layer "B.Cu") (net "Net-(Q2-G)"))
 (segment (start 81.89 80.13) (end 83.5 81.74) (width 1) (layer "B.Cu") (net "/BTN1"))
 (segment (start 95 79) (end 92.26 81.74) (width 1) (layer "B.Cu") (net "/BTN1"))
 (segment (start 81.89 77.28) (end 81.89 80.13) (width 1) (layer "B.Cu") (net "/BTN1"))
 (segment (start 83.5 81.74) (end 92.26 81.74) (width 1) (layer "B.Cu") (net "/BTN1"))
 (segment (start 95 58.25) (end 95 79) (width 1) (layer "B.Cu") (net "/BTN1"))
 (segment (start 91.75 55) (end 95 58.25) (width 1) (layer "B.Cu") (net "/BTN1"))
 (segment (start 98.25 78) (end 98.25 81.75) (width 1) (layer "B.Cu") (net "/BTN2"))
 (segment (start 82.26 84.5) (end 79.5 81.74) (width 1) (layer "B.Cu") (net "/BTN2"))
 (segment (start 95.5 84.5) (end 82.26 84.5) (width 1) (layer "B.Cu") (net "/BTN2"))
 (segment (start 79.35 81.59) (end 79.5 81.74) (width 1) (layer "B.Cu") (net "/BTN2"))
 (segment (start 79.35 77.28) (end 79.35 81.59) (width 1) (layer "B.Cu") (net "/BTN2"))
 (segment (start 98.25 81.75) (end 95.5 84.5) (width 1) (layer "B.Cu") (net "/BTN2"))
 (segment (start 54.5 82) (end 71.24 82) (width 1) (layer "B.Cu") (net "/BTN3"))
 (segment (start 52 79.5) (end 54.5 82) (width 1) (layer "B.Cu") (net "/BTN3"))
 (segment (start 52 58.25) (end 52 79.5) (width 1) (layer "B.Cu") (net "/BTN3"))
 (segment (start 74.27 77.28) (end 74.27 78.97) (width 1) (layer "B.Cu") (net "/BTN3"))
 (segment (start 74.27 78.97) (end 71.5 81.74) (width 1) (layer "B.Cu") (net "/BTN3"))
 (segment (start 48.75 55) (end 52 58.25) (width 1) (layer "B.Cu") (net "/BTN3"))
 (segment (start 71.24 82) (end 71.5 81.74) (width 1) (layer "B.Cu") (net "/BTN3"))
 (segment (start 48.75 80) (end 53.25 84.5) (width 1) (layer "B.Cu") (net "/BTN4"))
 (segment (start 53.25 84.5) (end 72.74 84.5) (width 1) (layer "B.Cu") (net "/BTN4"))
 (segment (start 48.75 78) (end 48.75 80) (width 1) (layer "B.Cu") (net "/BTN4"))
 (segment (start 76.81 80.43) (end 75.5 81.74) (width 1) (layer "B.Cu") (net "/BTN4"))
 (segment (start 72.74 84.5) (end 75.5 81.74) (width 1) (layer "B.Cu") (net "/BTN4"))
 (segment (start 76.81 77.28) (end 76.81 80.43) (width 1) (layer "B.Cu") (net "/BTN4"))
 (segment (start 74.27 96.73) (end 74.27 92.72) (width 1) (layer "B.Cu") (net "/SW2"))
 (segment (start 71.5 99.5) (end 74.27 96.73) (width 1) (layer "B.Cu") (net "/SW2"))
 (segment (start 41.5 95.54) (end 41.54 95.54) (width 1) (layer "B.Cu") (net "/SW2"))
 (segment (start 45.5 99.5) (end 71.5 99.5) (width 1) (layer "B.Cu") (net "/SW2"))
 (segment (start 41.54 95.54) (end 45.5 99.5) (width 1) (layer "B.Cu") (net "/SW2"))
 (segment (start 50.5 95.54) (end 51.46 96.5) (width 1) (layer "B.Cu") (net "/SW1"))
 (segment (start 51.46 96.5) (end 69.5 96.5) (width 1) (layer "B.Cu") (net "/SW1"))
 (segment (start 69.5 96.5) (end 71.73 94.27) (width 1) (layer "B.Cu") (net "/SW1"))
 (segment (start 71.73 94.27) (end 71.73 92.72) (width 1) (layer "B.Cu") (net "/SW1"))
 (segment (start 66 80) (end 59 80) (width 1) (layer "B.Cu") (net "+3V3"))
 (segment (start 55.25 73.5) (end 55.25 59.5) (width 1) (layer "B.Cu") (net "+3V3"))
 (segment (start 58.5 79.5) (end 58.5 76.75) (width 1) (layer "B.Cu") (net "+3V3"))
 (segment (start 70.43 73.5) (end 91.75 73.5) (width 1) (layer "B.Cu") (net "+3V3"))
 (segment (start 66.65 77.28) (end 66.65 79.35) (width 1) (layer "B.Cu") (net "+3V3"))
 (segment (start 59 80) (end 58.5 79.5) (width 1) (layer "B.Cu") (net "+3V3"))
 (segment (start 66.65 77.28) (end 70.43 73.5) (width 1) (layer "B.Cu") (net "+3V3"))
 (segment (start 66.65 79.35) (end 66 80) (width 1) (layer "B.Cu") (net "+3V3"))
 (segment (start 58.5 76.75) (end 55.25 73.5) (width 1) (layer "B.Cu") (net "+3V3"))
 (segment (start 91.75 73.5) (end 91.75 59.5) (width 1) (layer "B.Cu") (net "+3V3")))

